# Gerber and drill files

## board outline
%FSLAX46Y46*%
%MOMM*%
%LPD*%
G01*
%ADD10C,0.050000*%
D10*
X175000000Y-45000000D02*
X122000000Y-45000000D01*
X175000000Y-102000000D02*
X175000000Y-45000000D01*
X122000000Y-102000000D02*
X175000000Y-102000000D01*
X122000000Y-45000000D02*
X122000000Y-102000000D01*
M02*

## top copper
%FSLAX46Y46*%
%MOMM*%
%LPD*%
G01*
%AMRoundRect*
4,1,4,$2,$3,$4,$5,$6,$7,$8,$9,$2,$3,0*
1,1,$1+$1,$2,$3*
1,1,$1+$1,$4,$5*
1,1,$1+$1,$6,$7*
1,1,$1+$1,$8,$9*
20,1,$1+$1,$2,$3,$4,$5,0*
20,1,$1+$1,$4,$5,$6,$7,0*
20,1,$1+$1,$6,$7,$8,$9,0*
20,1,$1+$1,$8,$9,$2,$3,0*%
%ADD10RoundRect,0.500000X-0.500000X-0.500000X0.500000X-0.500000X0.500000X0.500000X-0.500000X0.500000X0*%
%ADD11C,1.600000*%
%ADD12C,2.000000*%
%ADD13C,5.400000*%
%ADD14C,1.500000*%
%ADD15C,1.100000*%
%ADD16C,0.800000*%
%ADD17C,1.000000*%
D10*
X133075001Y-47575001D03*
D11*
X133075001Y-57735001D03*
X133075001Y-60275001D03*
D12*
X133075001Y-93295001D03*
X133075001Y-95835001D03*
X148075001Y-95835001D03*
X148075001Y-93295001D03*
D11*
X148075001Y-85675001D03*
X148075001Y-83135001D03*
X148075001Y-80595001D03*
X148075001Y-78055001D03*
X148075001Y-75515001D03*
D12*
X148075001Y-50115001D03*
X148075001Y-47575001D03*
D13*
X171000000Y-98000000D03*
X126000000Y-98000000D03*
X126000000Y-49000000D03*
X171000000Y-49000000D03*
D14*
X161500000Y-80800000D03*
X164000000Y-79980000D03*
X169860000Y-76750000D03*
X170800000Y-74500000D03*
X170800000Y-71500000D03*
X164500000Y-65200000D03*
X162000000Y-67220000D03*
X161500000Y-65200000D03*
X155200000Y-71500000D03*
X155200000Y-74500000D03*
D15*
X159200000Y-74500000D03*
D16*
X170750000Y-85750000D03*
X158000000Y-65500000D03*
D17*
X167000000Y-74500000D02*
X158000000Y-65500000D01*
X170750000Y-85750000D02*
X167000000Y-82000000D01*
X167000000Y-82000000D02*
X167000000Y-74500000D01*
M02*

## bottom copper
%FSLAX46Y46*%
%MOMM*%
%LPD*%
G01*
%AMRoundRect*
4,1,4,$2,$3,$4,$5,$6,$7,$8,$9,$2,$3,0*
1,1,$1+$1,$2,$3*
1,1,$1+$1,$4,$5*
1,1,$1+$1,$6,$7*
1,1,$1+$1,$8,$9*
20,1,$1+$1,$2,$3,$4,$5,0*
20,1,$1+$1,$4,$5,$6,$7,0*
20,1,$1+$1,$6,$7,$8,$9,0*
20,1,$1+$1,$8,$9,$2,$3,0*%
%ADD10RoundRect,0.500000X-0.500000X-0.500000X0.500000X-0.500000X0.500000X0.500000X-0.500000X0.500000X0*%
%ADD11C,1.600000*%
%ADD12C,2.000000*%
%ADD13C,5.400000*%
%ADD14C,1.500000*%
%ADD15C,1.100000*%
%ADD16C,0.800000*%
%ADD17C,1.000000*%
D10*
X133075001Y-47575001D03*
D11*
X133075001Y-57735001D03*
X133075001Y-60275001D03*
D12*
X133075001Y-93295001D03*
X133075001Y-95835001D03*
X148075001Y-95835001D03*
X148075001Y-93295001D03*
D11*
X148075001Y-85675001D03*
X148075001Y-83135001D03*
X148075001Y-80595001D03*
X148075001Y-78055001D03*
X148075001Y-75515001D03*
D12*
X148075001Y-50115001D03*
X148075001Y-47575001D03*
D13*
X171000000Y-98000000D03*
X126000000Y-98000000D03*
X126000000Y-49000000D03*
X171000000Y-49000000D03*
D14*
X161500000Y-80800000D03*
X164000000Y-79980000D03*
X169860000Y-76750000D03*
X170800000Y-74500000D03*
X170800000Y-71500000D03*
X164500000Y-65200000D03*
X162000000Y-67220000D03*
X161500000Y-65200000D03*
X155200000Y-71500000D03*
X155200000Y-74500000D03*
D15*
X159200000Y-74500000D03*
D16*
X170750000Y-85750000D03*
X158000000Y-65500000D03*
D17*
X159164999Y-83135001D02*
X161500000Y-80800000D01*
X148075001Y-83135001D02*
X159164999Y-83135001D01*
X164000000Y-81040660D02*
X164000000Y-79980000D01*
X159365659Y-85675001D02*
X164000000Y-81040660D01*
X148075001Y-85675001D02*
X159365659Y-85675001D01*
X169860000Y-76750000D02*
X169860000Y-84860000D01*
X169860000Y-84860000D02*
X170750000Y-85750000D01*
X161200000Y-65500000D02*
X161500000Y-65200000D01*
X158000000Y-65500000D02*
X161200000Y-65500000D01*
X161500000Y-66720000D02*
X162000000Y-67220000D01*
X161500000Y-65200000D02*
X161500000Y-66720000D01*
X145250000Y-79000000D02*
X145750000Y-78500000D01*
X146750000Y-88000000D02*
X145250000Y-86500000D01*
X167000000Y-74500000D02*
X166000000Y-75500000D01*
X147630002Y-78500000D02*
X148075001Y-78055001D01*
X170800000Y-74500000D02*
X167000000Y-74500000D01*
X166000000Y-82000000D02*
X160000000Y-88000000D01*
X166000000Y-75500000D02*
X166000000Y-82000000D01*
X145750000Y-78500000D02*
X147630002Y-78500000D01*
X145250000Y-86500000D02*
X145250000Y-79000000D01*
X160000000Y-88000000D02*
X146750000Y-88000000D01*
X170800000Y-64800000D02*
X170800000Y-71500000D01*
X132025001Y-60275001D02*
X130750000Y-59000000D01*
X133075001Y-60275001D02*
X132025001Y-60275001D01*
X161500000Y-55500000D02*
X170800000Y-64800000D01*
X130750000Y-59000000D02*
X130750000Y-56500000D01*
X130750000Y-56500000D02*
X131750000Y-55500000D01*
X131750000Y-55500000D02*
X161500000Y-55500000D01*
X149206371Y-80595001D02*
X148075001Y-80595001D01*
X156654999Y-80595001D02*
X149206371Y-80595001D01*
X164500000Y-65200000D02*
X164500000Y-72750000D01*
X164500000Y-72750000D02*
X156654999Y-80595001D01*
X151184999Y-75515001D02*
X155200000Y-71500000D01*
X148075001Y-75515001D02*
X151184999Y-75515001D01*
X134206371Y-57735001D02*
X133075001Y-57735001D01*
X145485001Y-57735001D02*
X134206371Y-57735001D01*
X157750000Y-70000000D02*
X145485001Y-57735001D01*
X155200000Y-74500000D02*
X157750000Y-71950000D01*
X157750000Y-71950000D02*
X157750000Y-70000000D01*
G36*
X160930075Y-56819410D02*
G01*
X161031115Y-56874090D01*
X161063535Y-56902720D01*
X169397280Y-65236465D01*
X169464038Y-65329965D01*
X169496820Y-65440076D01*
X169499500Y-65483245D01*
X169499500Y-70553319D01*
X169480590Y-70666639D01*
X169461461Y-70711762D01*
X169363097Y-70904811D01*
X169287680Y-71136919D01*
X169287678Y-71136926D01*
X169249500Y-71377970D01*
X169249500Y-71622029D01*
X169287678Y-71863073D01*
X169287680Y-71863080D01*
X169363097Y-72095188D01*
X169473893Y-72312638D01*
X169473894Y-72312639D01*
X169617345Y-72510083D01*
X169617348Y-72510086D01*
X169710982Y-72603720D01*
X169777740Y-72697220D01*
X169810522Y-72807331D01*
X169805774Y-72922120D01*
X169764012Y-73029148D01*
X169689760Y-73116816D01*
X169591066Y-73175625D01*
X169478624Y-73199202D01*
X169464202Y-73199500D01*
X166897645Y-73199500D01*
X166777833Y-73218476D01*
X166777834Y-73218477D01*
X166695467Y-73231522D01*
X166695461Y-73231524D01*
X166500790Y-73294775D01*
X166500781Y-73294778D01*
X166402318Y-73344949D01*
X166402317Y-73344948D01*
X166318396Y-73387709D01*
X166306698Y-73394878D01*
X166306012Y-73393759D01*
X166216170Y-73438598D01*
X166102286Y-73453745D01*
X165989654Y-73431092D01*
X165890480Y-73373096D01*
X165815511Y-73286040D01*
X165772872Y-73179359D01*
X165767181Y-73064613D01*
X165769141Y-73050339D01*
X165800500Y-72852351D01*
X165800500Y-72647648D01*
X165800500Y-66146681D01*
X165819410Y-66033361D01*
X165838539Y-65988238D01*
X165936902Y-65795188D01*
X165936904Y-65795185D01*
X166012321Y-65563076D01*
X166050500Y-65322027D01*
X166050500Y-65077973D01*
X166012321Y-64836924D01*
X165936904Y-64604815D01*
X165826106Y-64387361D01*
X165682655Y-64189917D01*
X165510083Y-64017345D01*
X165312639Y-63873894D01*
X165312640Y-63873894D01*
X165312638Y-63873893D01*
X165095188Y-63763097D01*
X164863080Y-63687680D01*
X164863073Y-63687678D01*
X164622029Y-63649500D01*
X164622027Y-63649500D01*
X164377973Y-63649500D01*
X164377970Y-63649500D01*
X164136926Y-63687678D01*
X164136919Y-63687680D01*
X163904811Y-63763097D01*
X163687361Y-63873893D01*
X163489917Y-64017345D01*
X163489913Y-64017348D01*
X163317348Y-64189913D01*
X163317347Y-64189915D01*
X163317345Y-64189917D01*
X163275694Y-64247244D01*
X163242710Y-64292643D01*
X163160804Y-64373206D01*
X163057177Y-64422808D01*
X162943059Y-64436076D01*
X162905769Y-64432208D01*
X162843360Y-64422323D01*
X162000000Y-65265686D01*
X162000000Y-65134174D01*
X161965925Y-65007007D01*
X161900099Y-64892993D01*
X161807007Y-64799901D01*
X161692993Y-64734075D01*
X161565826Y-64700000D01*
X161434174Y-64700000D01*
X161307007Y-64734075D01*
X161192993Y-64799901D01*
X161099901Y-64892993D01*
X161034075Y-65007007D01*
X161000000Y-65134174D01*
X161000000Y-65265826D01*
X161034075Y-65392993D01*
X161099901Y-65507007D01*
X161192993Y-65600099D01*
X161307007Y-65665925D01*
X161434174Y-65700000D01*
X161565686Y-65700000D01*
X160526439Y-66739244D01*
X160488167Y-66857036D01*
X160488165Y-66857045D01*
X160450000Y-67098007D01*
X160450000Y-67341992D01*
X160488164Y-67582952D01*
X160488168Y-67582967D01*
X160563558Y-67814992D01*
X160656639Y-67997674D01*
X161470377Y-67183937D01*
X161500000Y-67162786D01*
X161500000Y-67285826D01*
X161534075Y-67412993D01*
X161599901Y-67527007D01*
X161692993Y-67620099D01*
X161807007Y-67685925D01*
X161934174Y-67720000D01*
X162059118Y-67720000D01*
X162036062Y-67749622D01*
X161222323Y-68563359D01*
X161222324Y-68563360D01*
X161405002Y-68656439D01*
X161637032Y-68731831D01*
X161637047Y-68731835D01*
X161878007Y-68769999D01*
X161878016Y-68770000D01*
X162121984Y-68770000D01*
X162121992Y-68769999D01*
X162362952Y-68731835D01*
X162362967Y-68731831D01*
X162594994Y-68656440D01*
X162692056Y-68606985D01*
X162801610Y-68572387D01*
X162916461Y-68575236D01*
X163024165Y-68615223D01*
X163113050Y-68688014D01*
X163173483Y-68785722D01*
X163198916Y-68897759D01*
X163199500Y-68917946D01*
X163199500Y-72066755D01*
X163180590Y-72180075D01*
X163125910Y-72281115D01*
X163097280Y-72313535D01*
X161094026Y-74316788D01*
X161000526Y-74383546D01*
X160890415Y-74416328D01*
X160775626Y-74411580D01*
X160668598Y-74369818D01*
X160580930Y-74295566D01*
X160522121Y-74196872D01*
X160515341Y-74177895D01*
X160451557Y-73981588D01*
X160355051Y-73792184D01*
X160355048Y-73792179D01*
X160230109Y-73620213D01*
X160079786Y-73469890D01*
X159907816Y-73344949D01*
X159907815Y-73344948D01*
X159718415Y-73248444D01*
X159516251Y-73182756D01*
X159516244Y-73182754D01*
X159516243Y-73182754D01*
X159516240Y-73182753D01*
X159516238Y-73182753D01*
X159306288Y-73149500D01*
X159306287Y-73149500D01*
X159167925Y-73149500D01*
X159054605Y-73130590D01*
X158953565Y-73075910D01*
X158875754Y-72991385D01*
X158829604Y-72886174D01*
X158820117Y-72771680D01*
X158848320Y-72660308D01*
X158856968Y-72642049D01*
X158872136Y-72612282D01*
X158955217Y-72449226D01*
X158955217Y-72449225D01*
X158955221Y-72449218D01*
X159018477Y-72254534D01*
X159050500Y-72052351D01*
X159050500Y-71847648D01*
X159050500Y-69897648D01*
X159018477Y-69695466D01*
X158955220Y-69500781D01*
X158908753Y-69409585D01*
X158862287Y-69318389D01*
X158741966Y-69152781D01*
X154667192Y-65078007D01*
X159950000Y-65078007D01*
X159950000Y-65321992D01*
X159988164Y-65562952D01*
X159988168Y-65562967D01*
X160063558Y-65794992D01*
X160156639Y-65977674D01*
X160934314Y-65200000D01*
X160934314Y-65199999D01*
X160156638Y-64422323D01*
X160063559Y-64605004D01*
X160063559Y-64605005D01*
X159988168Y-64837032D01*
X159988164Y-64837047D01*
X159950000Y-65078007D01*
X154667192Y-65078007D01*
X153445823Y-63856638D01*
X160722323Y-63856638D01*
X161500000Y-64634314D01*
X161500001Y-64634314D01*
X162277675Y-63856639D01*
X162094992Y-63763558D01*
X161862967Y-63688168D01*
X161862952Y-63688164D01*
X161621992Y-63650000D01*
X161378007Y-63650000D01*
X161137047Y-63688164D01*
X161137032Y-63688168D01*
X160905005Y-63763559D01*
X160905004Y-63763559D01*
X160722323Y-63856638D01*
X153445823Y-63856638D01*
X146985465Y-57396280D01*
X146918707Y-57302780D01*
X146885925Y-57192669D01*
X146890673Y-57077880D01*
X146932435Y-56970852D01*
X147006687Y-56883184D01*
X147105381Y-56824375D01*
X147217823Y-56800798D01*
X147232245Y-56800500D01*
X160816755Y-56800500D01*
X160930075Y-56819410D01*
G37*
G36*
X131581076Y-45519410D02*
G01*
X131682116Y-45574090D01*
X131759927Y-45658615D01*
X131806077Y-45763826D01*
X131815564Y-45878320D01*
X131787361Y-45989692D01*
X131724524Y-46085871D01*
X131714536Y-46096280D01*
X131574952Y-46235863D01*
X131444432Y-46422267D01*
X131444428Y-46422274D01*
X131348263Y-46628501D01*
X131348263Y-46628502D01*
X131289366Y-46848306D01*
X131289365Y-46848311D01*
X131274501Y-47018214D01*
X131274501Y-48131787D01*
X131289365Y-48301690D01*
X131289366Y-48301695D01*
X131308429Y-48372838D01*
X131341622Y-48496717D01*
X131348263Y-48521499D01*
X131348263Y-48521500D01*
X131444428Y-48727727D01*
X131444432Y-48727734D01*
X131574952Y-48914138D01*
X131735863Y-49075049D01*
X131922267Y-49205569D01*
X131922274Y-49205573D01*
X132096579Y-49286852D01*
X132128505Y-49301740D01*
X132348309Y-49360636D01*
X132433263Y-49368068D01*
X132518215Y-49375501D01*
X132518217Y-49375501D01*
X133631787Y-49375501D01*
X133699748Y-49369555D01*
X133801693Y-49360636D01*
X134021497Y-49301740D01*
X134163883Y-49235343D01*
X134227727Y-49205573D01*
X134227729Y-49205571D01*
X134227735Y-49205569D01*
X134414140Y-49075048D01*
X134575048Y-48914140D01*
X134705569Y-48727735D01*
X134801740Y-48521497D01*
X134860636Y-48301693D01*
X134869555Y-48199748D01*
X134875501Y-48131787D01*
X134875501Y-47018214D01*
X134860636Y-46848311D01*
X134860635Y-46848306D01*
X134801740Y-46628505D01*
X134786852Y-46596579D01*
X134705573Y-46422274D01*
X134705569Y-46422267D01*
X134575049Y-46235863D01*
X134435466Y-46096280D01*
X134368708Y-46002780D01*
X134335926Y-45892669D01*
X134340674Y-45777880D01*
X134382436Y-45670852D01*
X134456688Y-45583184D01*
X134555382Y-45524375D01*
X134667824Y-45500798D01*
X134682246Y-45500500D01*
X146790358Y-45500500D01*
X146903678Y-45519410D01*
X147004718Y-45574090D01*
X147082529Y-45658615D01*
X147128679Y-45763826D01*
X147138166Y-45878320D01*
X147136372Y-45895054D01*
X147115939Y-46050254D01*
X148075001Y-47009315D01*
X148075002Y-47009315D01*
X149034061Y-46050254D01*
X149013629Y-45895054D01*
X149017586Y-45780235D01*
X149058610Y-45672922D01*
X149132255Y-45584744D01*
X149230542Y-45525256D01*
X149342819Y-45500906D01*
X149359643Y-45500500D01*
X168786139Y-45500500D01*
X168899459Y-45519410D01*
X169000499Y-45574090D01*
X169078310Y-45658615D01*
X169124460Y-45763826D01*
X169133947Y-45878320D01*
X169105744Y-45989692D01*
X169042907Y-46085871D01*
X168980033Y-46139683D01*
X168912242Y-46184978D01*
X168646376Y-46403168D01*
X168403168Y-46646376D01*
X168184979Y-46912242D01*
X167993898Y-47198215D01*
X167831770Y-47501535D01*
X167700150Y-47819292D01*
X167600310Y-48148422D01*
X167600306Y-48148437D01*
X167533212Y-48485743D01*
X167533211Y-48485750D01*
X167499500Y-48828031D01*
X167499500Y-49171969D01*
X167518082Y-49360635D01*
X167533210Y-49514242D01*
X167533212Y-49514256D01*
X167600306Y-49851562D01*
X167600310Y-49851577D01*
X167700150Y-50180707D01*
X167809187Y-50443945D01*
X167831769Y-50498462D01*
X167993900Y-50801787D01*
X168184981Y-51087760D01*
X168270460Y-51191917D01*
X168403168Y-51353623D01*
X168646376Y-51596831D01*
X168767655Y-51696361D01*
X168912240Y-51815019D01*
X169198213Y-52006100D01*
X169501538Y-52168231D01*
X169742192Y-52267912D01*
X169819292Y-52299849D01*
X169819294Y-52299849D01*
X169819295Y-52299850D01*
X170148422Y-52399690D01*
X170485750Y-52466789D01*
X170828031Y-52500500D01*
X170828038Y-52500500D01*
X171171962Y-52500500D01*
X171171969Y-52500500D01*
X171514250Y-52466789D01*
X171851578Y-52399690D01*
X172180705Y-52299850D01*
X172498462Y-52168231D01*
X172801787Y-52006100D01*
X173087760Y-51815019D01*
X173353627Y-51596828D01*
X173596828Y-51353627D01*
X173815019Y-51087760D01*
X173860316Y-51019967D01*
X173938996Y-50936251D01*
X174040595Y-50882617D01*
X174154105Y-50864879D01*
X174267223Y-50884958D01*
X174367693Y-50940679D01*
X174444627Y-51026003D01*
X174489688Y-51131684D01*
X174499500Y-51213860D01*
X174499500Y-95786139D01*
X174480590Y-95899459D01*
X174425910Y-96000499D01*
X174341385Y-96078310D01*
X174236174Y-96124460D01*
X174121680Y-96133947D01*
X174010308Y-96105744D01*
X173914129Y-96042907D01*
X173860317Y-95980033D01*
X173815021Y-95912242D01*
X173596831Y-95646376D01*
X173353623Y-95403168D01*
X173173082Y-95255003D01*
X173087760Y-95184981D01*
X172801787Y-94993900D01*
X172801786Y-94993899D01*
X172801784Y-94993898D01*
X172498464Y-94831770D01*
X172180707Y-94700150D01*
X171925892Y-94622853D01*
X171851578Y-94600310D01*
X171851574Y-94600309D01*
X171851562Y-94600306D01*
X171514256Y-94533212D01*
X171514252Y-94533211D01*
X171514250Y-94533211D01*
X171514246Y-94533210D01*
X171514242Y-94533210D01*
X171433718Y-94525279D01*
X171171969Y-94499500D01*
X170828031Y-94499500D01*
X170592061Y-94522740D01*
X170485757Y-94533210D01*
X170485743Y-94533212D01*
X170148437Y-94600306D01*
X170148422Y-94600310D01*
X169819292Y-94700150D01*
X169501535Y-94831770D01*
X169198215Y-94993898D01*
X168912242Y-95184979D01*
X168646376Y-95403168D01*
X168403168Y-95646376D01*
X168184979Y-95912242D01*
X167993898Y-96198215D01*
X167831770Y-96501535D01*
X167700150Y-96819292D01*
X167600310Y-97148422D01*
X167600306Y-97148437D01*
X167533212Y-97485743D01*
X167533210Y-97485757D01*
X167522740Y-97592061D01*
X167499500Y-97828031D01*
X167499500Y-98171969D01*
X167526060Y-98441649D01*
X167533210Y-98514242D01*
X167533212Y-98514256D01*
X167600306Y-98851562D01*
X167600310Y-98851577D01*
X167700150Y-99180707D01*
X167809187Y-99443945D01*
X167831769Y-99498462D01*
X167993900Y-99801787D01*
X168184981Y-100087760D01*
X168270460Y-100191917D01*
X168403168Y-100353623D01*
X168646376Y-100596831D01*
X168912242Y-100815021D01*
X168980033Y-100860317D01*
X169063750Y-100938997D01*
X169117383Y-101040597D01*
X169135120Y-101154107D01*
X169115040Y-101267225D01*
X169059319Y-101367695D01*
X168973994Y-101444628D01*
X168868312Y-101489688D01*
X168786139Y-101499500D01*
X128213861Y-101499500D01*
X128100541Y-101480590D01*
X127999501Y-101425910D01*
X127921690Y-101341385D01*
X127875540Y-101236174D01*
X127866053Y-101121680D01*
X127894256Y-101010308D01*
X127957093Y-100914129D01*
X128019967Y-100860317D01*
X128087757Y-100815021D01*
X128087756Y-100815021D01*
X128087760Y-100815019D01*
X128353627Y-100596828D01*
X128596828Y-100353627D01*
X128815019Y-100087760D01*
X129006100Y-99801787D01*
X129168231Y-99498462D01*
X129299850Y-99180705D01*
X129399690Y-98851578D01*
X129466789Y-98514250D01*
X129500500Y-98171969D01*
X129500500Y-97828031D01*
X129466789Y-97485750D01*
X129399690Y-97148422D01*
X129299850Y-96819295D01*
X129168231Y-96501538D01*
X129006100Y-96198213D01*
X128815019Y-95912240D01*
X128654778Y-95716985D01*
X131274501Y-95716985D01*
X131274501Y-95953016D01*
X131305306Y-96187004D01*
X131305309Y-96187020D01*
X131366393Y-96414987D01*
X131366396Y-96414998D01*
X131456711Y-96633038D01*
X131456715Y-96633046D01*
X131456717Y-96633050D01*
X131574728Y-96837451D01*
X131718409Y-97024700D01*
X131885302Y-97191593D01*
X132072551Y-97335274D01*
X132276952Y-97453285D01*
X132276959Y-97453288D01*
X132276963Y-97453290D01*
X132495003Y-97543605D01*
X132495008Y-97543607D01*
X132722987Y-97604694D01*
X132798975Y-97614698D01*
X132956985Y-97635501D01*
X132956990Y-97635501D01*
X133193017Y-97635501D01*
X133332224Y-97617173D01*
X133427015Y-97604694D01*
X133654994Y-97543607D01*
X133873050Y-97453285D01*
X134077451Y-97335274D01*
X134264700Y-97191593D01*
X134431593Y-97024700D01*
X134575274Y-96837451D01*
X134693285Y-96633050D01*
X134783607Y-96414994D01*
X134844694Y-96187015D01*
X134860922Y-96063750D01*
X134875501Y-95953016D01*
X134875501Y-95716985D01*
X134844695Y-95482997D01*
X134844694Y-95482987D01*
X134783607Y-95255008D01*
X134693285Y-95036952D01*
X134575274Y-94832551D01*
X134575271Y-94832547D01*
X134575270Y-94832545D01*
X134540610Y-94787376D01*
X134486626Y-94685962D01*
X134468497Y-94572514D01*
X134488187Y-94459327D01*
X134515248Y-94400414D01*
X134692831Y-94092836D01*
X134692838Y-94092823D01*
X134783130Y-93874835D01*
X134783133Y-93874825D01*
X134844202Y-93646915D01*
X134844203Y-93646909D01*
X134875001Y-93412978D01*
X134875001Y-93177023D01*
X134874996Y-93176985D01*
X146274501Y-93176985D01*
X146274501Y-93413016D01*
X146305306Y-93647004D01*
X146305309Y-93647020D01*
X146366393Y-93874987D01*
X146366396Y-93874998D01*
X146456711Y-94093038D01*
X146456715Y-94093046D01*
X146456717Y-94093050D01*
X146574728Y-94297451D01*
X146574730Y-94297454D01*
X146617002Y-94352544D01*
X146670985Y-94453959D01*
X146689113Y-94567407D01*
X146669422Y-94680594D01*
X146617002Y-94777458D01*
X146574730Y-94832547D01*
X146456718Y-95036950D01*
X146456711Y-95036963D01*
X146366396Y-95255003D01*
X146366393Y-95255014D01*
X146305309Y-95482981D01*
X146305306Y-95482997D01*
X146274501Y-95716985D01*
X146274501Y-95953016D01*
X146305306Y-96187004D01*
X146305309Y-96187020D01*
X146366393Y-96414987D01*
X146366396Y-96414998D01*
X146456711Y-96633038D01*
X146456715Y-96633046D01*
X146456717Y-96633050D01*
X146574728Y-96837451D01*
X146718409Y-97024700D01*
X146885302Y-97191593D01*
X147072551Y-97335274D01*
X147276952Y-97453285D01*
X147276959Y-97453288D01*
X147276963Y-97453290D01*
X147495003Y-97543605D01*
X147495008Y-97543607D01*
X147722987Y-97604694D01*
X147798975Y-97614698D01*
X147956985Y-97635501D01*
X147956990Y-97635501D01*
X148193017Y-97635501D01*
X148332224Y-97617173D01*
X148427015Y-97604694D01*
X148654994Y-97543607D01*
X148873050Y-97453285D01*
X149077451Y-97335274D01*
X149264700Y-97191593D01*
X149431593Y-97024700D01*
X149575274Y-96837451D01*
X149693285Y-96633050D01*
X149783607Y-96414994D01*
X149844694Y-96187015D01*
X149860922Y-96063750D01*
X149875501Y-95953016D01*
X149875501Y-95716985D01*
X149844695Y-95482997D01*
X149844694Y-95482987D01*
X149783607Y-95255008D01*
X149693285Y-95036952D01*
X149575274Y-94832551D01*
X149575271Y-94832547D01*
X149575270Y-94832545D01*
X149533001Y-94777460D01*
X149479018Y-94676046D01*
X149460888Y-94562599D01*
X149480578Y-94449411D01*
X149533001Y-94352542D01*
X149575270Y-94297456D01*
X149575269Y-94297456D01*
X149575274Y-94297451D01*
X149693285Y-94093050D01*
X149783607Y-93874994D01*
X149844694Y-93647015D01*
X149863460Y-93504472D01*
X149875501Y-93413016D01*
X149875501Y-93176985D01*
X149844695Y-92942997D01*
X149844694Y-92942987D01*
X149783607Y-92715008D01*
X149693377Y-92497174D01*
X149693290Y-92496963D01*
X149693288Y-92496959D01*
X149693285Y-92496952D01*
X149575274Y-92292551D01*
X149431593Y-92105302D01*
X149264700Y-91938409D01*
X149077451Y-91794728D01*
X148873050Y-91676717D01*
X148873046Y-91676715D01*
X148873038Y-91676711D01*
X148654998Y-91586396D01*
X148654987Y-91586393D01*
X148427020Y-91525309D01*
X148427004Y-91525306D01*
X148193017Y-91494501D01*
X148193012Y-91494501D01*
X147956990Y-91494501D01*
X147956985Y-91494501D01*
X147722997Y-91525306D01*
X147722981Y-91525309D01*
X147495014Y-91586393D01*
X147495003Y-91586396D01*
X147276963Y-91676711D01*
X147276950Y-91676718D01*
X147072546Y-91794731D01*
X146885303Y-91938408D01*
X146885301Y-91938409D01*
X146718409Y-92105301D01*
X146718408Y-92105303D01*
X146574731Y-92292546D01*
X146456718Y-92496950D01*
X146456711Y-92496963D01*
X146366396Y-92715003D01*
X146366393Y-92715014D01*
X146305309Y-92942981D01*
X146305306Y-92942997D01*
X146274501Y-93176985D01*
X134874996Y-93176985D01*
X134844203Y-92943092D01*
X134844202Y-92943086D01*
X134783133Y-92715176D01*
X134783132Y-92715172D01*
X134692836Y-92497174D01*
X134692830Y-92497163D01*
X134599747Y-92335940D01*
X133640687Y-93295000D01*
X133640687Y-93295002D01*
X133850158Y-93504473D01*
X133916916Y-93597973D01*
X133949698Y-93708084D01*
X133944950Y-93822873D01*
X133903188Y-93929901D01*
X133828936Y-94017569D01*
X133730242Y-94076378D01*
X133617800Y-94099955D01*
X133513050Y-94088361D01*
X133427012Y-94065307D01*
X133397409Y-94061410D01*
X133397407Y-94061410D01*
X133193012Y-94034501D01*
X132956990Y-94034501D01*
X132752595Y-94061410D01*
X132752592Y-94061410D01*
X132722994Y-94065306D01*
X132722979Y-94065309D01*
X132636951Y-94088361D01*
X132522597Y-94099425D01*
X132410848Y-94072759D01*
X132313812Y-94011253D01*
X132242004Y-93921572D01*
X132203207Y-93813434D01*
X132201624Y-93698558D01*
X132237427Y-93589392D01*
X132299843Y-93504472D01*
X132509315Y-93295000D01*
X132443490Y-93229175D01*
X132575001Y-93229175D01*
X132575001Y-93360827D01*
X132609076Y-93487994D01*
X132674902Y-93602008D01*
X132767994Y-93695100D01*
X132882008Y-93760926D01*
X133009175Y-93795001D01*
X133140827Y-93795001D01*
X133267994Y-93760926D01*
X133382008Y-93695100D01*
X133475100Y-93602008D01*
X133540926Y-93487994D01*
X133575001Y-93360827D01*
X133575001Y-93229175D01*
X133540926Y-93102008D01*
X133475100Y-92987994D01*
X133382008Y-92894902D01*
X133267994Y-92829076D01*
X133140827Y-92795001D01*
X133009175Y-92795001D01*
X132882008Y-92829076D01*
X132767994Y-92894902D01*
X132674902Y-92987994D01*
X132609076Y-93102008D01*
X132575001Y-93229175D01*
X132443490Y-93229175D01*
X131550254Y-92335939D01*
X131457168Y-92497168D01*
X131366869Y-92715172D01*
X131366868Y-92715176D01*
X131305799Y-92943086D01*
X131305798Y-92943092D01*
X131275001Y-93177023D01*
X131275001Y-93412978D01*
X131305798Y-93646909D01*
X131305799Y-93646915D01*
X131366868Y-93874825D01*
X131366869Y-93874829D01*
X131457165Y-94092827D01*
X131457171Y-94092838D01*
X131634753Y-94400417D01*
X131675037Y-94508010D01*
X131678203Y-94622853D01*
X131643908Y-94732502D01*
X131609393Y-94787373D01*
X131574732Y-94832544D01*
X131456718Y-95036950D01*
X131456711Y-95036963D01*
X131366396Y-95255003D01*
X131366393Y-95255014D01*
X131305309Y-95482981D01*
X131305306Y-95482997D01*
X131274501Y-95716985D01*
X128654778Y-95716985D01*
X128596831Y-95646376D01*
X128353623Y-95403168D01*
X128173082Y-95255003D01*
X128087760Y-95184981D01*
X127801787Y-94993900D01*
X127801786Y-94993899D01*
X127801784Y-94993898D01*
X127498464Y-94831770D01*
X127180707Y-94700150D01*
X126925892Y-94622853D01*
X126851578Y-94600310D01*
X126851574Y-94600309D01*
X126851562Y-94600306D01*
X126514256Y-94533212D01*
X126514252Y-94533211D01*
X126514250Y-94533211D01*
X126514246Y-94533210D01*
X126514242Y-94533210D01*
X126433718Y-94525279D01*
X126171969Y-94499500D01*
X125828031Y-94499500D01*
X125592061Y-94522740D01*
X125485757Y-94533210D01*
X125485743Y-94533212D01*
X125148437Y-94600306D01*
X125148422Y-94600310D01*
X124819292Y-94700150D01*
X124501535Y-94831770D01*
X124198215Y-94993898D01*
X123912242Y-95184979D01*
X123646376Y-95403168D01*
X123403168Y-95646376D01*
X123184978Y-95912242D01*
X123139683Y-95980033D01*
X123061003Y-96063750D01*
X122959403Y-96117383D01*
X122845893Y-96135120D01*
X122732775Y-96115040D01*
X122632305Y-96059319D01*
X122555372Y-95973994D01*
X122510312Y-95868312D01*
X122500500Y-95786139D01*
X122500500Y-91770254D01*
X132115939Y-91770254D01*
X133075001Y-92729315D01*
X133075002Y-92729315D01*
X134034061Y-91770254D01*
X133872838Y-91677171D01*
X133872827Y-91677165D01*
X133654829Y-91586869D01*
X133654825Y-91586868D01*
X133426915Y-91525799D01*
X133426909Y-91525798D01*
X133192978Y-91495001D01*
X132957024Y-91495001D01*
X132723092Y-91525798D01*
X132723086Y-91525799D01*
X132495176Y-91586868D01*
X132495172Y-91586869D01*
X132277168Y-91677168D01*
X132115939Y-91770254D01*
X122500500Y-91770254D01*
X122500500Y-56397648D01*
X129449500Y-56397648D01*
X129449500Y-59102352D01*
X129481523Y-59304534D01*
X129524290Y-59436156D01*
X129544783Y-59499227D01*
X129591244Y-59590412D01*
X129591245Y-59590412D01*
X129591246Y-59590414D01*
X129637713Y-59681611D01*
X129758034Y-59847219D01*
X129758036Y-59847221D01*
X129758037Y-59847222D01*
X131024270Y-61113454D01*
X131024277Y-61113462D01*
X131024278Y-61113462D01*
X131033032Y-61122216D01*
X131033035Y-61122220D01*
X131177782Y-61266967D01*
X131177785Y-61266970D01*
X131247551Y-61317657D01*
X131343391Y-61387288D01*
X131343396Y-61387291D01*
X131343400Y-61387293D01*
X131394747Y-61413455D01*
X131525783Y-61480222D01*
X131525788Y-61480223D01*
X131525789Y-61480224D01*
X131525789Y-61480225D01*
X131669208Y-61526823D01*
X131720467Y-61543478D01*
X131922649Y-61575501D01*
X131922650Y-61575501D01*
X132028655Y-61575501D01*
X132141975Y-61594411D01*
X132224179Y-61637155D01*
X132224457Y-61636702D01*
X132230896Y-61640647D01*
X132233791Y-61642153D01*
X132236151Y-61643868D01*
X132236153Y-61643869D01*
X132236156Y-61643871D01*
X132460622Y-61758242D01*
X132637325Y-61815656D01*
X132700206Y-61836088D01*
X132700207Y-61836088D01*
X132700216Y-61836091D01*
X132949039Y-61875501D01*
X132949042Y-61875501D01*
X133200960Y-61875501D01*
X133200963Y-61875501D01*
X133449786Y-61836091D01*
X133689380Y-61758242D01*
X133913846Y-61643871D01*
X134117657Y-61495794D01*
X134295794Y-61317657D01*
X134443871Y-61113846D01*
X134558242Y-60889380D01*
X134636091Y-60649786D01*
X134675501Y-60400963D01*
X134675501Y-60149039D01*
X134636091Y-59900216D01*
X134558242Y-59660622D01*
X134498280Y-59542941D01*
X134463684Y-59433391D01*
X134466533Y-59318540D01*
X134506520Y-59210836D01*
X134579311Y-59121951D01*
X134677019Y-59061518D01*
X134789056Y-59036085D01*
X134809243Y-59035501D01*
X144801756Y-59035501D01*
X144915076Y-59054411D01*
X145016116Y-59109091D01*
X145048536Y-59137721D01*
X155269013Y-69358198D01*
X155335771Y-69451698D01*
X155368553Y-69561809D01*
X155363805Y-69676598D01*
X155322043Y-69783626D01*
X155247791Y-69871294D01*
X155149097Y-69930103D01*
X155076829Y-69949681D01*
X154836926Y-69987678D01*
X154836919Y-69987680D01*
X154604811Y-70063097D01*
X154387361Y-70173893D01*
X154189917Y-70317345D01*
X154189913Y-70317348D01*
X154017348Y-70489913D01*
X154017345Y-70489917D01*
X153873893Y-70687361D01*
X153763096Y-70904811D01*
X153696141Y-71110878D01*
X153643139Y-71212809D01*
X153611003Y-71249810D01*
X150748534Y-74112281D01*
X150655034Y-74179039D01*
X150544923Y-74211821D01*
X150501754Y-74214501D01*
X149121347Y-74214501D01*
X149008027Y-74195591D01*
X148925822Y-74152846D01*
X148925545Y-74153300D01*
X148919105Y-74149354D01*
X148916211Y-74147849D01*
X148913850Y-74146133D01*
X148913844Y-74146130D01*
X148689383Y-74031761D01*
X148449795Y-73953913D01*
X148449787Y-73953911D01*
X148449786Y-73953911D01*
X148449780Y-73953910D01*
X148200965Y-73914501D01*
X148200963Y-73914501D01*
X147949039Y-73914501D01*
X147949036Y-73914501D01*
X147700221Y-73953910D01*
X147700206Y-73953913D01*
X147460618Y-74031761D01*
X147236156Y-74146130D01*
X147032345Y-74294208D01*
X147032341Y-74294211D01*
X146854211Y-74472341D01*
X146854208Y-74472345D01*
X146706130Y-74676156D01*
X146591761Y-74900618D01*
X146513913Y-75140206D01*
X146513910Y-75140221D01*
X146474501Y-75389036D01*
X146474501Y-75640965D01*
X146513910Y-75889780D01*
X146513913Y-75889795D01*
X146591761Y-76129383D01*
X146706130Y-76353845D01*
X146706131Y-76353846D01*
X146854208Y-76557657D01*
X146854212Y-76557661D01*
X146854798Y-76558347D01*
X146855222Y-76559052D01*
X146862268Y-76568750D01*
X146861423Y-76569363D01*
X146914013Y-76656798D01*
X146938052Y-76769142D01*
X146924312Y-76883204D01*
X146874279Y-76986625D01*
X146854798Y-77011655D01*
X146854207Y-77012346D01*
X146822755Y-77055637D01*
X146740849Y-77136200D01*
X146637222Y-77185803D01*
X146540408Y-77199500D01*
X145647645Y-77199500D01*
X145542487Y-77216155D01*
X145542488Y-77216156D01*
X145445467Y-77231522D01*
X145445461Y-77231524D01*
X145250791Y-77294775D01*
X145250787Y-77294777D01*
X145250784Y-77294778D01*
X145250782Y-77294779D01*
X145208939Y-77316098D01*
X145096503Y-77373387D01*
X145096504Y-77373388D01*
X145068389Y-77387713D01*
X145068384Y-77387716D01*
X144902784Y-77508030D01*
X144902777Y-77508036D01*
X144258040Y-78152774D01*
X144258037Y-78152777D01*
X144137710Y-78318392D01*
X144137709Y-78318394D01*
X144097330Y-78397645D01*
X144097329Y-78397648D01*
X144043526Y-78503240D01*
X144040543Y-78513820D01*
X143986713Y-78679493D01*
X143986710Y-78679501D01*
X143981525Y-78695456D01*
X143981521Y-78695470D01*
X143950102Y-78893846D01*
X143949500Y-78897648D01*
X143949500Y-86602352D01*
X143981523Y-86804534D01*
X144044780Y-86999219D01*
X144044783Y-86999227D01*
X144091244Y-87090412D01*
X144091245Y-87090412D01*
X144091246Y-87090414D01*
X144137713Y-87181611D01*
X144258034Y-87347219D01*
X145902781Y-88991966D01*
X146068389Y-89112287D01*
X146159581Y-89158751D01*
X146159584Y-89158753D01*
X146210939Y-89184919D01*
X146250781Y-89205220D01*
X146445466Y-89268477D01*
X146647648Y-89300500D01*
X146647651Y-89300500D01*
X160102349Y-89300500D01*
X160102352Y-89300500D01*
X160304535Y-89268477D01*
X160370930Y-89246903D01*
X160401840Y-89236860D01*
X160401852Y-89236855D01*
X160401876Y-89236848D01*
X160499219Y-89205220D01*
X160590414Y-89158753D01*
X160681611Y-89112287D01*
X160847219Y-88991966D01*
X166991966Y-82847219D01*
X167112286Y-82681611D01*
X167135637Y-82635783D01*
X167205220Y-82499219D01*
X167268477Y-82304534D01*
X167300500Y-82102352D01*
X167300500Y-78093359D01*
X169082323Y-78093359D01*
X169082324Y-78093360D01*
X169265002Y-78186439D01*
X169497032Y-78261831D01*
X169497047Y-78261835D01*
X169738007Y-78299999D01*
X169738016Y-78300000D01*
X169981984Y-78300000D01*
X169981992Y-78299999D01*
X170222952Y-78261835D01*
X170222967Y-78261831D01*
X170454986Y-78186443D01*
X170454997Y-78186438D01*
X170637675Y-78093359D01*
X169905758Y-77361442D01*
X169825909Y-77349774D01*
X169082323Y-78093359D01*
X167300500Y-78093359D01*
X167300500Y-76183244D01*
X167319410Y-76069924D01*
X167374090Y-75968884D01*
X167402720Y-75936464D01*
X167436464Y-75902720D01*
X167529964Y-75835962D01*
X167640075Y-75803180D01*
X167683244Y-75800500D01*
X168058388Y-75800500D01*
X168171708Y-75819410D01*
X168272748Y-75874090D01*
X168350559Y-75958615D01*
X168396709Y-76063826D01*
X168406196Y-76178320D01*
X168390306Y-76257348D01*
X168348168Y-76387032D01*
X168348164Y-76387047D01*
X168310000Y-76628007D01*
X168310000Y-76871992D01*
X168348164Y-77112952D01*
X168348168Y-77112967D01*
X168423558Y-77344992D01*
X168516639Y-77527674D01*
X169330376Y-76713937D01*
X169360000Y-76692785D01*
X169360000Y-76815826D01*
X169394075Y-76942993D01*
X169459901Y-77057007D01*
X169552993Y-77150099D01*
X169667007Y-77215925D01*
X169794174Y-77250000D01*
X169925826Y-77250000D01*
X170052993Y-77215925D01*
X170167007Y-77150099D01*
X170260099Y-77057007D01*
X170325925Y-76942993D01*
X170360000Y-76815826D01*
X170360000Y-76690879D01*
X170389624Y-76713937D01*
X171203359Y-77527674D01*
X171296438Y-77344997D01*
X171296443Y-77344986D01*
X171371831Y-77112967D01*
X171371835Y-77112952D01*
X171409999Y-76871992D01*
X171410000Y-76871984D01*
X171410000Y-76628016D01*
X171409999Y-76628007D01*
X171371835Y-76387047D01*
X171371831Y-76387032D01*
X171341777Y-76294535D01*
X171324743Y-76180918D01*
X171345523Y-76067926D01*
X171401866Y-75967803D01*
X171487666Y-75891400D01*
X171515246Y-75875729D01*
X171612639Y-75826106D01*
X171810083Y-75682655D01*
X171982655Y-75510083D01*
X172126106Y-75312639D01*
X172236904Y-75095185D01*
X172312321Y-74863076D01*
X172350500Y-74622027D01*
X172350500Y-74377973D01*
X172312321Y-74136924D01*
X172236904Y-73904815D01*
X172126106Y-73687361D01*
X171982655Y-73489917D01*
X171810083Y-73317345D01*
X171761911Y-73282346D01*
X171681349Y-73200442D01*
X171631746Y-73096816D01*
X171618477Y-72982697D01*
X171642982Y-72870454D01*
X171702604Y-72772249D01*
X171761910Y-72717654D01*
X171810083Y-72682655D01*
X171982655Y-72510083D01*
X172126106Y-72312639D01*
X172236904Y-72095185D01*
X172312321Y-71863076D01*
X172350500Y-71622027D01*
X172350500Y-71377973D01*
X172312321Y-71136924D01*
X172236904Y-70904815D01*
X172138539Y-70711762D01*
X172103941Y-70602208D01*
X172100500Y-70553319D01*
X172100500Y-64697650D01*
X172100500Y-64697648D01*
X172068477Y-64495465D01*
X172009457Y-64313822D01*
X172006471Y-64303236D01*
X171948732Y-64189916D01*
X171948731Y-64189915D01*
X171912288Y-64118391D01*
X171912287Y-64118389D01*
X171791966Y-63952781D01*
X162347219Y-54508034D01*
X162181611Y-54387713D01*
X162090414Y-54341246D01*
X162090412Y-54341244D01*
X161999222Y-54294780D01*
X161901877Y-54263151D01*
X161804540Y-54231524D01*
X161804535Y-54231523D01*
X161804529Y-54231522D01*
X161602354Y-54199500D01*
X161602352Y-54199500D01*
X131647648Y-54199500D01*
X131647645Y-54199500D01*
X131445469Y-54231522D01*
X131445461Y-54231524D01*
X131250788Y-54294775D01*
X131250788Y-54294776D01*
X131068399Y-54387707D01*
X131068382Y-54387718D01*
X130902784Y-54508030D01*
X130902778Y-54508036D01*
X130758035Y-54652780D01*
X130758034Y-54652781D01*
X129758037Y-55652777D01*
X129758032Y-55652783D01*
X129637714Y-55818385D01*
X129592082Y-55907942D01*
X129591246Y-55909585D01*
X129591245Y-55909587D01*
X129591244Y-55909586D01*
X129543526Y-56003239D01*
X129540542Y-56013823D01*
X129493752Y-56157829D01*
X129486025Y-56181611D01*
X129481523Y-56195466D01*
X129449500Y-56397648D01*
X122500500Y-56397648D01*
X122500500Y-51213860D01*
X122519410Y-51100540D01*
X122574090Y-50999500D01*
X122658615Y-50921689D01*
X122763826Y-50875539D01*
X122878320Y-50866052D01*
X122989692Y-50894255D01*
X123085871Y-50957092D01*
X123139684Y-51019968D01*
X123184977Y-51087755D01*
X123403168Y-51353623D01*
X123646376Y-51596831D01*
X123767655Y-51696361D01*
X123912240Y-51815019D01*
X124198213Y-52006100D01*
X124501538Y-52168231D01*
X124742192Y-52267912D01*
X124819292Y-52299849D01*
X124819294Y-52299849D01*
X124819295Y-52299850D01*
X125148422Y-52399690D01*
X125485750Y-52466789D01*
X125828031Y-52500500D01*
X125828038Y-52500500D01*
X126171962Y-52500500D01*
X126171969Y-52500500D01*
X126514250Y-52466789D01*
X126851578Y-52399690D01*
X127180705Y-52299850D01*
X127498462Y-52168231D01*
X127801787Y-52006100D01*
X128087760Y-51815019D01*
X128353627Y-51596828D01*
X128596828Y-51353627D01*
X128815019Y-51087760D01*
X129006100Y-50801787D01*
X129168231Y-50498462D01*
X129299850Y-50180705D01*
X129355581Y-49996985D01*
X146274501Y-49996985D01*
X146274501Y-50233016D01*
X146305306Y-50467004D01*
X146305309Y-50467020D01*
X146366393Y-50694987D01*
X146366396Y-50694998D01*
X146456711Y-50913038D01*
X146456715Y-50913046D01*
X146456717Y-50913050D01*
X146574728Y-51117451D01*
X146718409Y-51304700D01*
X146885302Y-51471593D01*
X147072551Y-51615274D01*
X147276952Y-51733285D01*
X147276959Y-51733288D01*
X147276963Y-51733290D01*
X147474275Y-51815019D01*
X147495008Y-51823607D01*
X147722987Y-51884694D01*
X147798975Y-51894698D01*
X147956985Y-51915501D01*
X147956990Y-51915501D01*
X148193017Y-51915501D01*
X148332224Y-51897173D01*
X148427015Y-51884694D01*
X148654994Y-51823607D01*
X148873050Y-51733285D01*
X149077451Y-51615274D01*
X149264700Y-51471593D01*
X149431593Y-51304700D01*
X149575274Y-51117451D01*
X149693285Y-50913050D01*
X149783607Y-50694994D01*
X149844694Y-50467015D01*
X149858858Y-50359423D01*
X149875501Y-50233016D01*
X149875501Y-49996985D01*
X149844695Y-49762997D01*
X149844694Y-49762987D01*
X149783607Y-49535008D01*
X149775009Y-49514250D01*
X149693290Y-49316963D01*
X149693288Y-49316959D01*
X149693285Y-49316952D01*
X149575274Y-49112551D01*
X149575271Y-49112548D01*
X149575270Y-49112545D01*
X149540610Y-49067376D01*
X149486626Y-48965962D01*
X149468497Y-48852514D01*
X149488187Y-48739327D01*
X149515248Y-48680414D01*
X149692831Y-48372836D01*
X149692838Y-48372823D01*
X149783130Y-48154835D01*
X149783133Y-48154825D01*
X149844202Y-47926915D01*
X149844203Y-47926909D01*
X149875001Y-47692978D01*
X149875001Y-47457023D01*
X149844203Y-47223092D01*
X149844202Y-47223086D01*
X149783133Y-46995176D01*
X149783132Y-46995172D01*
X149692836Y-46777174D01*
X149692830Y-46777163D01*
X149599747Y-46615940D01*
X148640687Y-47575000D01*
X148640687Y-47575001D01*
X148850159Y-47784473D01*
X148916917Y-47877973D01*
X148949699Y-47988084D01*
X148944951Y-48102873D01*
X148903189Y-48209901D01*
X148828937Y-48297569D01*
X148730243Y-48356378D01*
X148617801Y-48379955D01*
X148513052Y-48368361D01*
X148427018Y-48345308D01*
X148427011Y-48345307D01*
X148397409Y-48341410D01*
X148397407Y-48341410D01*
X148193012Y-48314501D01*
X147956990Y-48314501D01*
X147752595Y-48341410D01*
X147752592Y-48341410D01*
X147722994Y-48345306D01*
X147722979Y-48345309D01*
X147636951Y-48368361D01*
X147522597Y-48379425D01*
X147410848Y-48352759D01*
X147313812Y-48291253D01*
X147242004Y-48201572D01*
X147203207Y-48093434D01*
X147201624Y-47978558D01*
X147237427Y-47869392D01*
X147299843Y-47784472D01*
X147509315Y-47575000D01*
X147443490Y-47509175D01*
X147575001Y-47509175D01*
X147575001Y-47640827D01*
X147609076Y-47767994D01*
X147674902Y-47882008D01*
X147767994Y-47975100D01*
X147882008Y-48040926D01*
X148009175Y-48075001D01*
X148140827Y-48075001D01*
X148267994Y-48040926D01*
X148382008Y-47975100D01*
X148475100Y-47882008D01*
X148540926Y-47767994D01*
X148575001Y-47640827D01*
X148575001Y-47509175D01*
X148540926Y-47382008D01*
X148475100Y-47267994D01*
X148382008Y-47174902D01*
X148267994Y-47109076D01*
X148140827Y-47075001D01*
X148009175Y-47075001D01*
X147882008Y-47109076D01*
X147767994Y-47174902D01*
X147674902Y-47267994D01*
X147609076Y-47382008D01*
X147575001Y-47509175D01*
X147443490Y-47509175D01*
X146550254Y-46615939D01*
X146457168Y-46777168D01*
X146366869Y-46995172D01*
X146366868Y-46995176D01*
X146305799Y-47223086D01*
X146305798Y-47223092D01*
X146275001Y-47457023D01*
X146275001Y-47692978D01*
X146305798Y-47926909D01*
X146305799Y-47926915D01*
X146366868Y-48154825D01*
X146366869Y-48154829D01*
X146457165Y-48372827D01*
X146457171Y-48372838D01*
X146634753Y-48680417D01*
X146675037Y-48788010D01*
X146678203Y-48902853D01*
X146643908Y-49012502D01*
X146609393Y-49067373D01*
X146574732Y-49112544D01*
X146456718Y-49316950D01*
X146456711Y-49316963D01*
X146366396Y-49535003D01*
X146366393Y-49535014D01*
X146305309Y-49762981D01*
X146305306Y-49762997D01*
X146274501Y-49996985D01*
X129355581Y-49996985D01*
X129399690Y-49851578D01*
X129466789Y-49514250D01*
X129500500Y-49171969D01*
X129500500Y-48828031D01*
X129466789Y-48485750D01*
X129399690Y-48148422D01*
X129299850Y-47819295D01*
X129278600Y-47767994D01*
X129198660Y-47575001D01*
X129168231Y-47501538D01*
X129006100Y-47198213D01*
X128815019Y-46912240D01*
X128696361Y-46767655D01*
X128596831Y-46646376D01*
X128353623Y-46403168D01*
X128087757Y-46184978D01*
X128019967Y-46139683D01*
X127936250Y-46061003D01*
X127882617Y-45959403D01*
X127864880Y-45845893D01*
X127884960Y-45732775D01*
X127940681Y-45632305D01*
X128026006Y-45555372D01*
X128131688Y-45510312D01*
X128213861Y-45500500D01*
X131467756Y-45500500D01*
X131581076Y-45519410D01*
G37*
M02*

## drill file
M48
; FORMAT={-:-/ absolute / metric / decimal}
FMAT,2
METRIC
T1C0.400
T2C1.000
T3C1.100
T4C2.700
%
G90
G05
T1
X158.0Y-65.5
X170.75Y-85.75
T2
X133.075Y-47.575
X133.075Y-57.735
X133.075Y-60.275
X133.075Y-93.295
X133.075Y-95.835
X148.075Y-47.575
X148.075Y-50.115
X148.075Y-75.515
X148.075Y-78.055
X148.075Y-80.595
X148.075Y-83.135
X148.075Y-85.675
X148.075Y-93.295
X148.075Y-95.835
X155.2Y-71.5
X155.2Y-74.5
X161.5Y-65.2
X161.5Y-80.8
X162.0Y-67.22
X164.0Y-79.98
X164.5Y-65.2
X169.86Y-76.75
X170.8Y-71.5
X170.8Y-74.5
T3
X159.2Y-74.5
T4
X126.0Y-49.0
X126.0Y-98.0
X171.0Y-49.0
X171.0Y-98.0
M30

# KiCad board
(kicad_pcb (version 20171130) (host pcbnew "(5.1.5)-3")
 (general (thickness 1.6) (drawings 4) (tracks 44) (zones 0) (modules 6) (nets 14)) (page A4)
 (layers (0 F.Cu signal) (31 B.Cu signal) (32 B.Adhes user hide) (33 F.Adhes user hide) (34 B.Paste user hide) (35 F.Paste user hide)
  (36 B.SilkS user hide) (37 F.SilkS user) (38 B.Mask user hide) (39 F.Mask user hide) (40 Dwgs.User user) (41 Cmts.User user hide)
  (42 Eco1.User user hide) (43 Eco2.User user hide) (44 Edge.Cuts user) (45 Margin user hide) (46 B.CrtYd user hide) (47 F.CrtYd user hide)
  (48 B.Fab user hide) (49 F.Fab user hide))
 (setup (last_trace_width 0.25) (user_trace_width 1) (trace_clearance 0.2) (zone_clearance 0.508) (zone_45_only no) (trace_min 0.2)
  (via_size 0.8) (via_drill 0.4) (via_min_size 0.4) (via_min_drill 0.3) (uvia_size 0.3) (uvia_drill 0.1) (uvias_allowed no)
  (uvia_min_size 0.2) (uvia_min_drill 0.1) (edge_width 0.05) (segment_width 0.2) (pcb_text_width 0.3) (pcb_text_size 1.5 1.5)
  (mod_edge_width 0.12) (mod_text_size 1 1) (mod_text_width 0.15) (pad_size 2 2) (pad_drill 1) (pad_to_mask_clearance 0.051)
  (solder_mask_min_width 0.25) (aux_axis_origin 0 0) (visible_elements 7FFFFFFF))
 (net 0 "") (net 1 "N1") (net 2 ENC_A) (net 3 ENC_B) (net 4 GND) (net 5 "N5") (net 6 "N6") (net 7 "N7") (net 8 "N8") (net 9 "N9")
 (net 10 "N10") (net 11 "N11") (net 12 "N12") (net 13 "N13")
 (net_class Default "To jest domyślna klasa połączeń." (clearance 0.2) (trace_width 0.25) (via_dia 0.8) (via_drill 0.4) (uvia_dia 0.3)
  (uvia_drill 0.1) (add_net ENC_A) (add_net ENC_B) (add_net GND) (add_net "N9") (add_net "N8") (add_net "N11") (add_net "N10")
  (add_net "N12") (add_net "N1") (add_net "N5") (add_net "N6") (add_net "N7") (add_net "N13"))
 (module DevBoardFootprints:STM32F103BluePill (layer F.Cu) (at 140.575001 71.575001)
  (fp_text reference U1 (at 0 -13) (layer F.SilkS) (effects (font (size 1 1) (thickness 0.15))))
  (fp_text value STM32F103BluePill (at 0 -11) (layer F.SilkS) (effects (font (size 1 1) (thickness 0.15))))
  (pad 1 thru_hole roundrect (at -7.5 -24) (size 2 2) (drill 1) (layers *.Cu *.Mask) (roundrect_rratio 0.25) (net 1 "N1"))
  (pad 5 thru_hole circle (at -7.5 -13.84) (size 1.6 1.6) (drill 1) (layers *.Cu *.Mask) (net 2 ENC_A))
  (pad 6 thru_hole circle (at -7.5 -11.3) (size 1.6 1.6) (drill 1) (layers *.Cu *.Mask) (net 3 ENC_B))
  (pad 19 thru_hole circle (at -7.5 21.72) (size 2 2) (drill 1) (layers *.Cu *.Mask) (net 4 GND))
  (pad 20 thru_hole circle (at -7.5 24.26) (size 2 2) (drill 1) (layers *.Cu *.Mask) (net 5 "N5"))
  (pad 21 thru_hole circle (at 7.5 24.26) (size 2 2) (drill 1) (layers *.Cu *.Mask) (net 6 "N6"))
  (pad 22 thru_hole circle (at 7.5 21.72) (size 2 2) (drill 1) (layers *.Cu *.Mask) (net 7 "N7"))
  (pad 25 thru_hole circle (at 7.5 14.1) (size 1.6 1.6) (drill 1) (layers *.Cu *.Mask) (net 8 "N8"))
  (pad 26 thru_hole circle (at 7.5 11.56) (size 1.6 1.6) (drill 1) (layers *.Cu *.Mask) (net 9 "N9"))
  (pad 27 thru_hole circle (at 7.5 9.02) (size 1.6 1.6) (drill 1) (layers *.Cu *.Mask) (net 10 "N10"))
  (pad 28 thru_hole circle (at 7.5 6.48) (size 1.6 1.6) (drill 1) (layers *.Cu *.Mask) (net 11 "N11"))
  (pad 29 thru_hole circle (at 7.5 3.94) (size 1.6 1.6) (drill 1) (layers *.Cu *.Mask) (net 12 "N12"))
  (pad 39 thru_hole circle (at 7.5 -21.46) (size 2 2) (drill 1) (layers *.Cu *.Mask) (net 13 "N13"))
  (pad 40 thru_hole circle (at 7.5 -24) (size 2 2) (drill 1) (layers *.Cu *.Mask) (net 4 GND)))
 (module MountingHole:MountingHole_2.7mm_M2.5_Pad (layer F.Cu) (at 171 98)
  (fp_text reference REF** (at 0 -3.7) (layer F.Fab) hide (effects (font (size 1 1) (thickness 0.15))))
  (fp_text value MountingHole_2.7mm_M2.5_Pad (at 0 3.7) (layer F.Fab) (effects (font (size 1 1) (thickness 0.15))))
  (pad "" thru_hole circle (at 0 0) (size 5.4 5.4) (drill 2.7) (layers *.Cu *.Mask)))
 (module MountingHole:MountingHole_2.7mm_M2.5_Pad (layer F.Cu) (at 126 98)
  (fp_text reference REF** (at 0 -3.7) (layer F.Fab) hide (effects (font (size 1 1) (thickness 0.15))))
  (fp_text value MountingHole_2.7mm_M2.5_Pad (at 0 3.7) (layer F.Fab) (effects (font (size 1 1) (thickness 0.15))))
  (pad "" thru_hole circle (at 0 0) (size 5.4 5.4) (drill 2.7) (layers *.Cu *.Mask)))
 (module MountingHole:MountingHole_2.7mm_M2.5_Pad (layer F.Cu) (at 126 49)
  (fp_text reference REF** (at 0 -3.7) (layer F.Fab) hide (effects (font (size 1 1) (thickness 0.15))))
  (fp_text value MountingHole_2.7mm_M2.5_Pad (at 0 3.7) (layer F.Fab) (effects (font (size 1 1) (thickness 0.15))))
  (pad "" thru_hole circle (at 0 0) (size 5.4 5.4) (drill 2.7) (layers *.Cu *.Mask)))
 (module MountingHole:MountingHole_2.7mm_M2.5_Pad (layer F.Cu) (at 171 49)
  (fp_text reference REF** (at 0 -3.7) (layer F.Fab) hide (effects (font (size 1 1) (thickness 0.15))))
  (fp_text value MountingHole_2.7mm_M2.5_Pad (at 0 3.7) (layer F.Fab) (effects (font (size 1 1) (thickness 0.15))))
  (pad "" thru_hole circle (at 0 0) (size 5.4 5.4) (drill 2.7) (layers *.Cu *.Mask)))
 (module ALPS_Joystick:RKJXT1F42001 (layer F.Cu) (at 163 73)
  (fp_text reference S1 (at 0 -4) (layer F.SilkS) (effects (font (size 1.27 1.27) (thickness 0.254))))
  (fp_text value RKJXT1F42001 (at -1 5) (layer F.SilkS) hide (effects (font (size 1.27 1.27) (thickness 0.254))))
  (pad 1 thru_hole circle (at -1.5 7.8 90) (size 1.5 1.5) (drill 1) (layers *.Cu *.Mask) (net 9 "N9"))
  (pad 2 thru_hole circle (at 1 6.98 90) (size 1.5 1.5) (drill 1) (layers *.Cu *.Mask) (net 8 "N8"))
  (pad 3 thru_hole circle (at 6.86 3.75 90) (size 1.5 1.5) (drill 1) (layers *.Cu *.Mask) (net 4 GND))
  (pad 4 thru_hole circle (at 7.8 1.5 90) (size 1.5 1.5) (drill 1) (layers *.Cu *.Mask) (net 11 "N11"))
  (pad 5 thru_hole circle (at 7.8 -1.5 90) (size 1.5 1.5) (drill 1) (layers *.Cu *.Mask) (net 3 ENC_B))
  (pad 6 thru_hole circle (at 1.5 -7.8 90) (size 1.5 1.5) (drill 1) (layers *.Cu *.Mask) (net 10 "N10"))
  (pad 7 thru_hole circle (at -1 -5.78 90) (size 1.5 1.5) (drill 1) (layers *.Cu *.Mask) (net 4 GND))
  (pad 8 thru_hole circle (at -1.5 -7.8 90) (size 1.5 1.5) (drill 1) (layers *.Cu *.Mask) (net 4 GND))
  (pad 9 thru_hole circle (at -7.8 -1.5 90) (size 1.5 1.5) (drill 1) (layers *.Cu *.Mask) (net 12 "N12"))
  (pad 10 thru_hole circle (at -7.8 1.5 90) (size 1.5 1.5) (drill 1) (layers *.Cu *.Mask) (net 2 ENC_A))
  (pad "" thru_hole circle (at -3.8 1.5 90) (size 1.1 1.1) (drill 1.1) (layers *.Cu *.Mask)))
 (gr_line (start 175 45) (end 122 45) (layer Edge.Cuts) (width 0.05))
 (gr_line (start 175 102) (end 175 45) (layer Edge.Cuts) (width 0.05))
 (gr_line (start 122 102) (end 175 102) (layer Edge.Cuts) (width 0.05))
 (gr_line (start 122 45) (end 122 102) (layer Edge.Cuts) (width 0.05))
 (segment (start 159.164999 83.135001) (end 161.5 80.8) (width 1) (layer B.Cu) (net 9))
 (segment (start 148.075001 83.135001) (end 159.164999 83.135001) (width 1) (layer B.Cu) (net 9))
 (segment (start 164 81.04066) (end 164 79.98) (width 1) (layer B.Cu) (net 8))
 (segment (start 159.365659 85.675001) (end 164 81.04066) (width 1) (layer B.Cu) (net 8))
 (segment (start 148.075001 85.675001) (end 159.365659 85.675001) (width 1) (layer B.Cu) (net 8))
 (segment (start 169.86 76.75) (end 169.86 84.86) (width 1) (layer B.Cu) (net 4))
 (via (at 170.75 85.75) (size 0.8) (drill 0.4) (layers F.Cu B.Cu) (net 4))
 (segment (start 169.86 84.86) (end 170.75 85.75) (width 1) (layer B.Cu) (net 4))
 (via (at 158 65.5) (size 0.8) (drill 0.4) (layers F.Cu B.Cu) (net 4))
 (segment (start 161.2 65.5) (end 161.5 65.2) (width 1) (layer B.Cu) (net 4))
 (segment (start 158 65.5) (end 161.2 65.5) (width 1) (layer B.Cu) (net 4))
 (segment (start 161.5 66.72) (end 162 67.22) (width 1) (layer B.Cu) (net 4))
 (segment (start 161.5 65.2) (end 161.5 66.72) (width 1) (layer B.Cu) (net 4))
 (segment (start 167 74.5) (end 158 65.5) (width 1) (layer F.Cu) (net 4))
 (segment (start 170.75 85.75) (end 167 82) (width 1) (layer F.Cu) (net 4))
 (segment (start 167 82) (end 167 74.5) (width 1) (layer F.Cu) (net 4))
 (segment (start 145.25 79) (end 145.75 78.5) (width 1) (layer B.Cu) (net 11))
 (segment (start 146.75 88) (end 145.25 86.5) (width 1) (layer B.Cu) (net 11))
 (segment (start 167 74.5) (end 166 75.5) (width 1) (layer B.Cu) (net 11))
 (segment (start 147.630002 78.5) (end 148.075001 78.055001) (width 1) (layer B.Cu) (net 11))
 (segment (start 170.8 74.5) (end 167 74.5) (width 1) (layer B.Cu) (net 11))
 (segment (start 166 82) (end 160 88) (width 1) (layer B.Cu) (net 11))
 (segment (start 166 75.5) (end 166 82) (width 1) (layer B.Cu) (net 11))
 (segment (start 145.75 78.5) (end 147.630002 78.5) (width 1) (layer B.Cu) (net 11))
 (segment (start 145.25 86.5) (end 145.25 79) (width 1) (layer B.Cu) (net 11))
 (segment (start 160 88) (end 146.75 88) (width 1) (layer B.Cu) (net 11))
 (segment (start 170.8 64.8) (end 170.8 71.5) (width 1) (layer B.Cu) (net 3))
 (segment (start 132.025001 60.275001) (end 130.75 59) (width 1) (layer B.Cu) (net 3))
 (segment (start 133.075001 60.275001) (end 132.025001 60.275001) (width 1) (layer B.Cu) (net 3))
 (segment (start 161.5 55.5) (end 170.8 64.8) (width 1) (layer B.Cu) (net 3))
 (segment (start 130.75 59) (end 130.75 56.5) (width 1) (layer B.Cu) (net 3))
 (segment (start 130.75 56.5) (end 131.75 55.5) (width 1) (layer B.Cu) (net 3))
 (segment (start 131.75 55.5) (end 161.5 55.5) (width 1) (layer B.Cu) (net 3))
 (segment (start 149.206371 80.595001) (end 148.075001 80.595001) (width 1) (layer B.Cu) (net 10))
 (segment (start 156.654999 80.595001) (end 149.206371 80.595001) (width 1) (layer B.Cu) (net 10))
 (segment (start 164.5 65.2) (end 164.5 72.75) (width 1) (layer B.Cu) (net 10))
 (segment (start 164.5 72.75) (end 156.654999 80.595001) (width 1) (layer B.Cu) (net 10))
 (segment (start 151.184999 75.515001) (end 155.2 71.5) (width 1) (layer B.Cu) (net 12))
 (segment (start 148.075001 75.515001) (end 151.184999 75.515001) (width 1) (layer B.Cu) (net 12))
 (segment (start 134.206371 57.735001) (end 133.075001 57.735001) (width 1) (layer B.Cu) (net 2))
 (segment (start 145.485001 57.735001) (end 134.206371 57.735001) (width 1) (layer B.Cu) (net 2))
 (segment (start 157.75 70) (end 145.485001 57.735001) (width 1) (layer B.Cu) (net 2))
 (segment (start 155.2 74.5) (end 157.75 71.95) (width 1) (layer B.Cu) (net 2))
 (segment (start 157.75 71.95) (end 157.75 70) (width 1) (layer B.Cu) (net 2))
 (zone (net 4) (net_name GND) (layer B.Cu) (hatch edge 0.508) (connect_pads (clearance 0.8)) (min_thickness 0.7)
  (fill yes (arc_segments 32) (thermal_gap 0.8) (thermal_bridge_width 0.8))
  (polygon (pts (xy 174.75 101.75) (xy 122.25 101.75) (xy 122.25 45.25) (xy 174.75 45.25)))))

